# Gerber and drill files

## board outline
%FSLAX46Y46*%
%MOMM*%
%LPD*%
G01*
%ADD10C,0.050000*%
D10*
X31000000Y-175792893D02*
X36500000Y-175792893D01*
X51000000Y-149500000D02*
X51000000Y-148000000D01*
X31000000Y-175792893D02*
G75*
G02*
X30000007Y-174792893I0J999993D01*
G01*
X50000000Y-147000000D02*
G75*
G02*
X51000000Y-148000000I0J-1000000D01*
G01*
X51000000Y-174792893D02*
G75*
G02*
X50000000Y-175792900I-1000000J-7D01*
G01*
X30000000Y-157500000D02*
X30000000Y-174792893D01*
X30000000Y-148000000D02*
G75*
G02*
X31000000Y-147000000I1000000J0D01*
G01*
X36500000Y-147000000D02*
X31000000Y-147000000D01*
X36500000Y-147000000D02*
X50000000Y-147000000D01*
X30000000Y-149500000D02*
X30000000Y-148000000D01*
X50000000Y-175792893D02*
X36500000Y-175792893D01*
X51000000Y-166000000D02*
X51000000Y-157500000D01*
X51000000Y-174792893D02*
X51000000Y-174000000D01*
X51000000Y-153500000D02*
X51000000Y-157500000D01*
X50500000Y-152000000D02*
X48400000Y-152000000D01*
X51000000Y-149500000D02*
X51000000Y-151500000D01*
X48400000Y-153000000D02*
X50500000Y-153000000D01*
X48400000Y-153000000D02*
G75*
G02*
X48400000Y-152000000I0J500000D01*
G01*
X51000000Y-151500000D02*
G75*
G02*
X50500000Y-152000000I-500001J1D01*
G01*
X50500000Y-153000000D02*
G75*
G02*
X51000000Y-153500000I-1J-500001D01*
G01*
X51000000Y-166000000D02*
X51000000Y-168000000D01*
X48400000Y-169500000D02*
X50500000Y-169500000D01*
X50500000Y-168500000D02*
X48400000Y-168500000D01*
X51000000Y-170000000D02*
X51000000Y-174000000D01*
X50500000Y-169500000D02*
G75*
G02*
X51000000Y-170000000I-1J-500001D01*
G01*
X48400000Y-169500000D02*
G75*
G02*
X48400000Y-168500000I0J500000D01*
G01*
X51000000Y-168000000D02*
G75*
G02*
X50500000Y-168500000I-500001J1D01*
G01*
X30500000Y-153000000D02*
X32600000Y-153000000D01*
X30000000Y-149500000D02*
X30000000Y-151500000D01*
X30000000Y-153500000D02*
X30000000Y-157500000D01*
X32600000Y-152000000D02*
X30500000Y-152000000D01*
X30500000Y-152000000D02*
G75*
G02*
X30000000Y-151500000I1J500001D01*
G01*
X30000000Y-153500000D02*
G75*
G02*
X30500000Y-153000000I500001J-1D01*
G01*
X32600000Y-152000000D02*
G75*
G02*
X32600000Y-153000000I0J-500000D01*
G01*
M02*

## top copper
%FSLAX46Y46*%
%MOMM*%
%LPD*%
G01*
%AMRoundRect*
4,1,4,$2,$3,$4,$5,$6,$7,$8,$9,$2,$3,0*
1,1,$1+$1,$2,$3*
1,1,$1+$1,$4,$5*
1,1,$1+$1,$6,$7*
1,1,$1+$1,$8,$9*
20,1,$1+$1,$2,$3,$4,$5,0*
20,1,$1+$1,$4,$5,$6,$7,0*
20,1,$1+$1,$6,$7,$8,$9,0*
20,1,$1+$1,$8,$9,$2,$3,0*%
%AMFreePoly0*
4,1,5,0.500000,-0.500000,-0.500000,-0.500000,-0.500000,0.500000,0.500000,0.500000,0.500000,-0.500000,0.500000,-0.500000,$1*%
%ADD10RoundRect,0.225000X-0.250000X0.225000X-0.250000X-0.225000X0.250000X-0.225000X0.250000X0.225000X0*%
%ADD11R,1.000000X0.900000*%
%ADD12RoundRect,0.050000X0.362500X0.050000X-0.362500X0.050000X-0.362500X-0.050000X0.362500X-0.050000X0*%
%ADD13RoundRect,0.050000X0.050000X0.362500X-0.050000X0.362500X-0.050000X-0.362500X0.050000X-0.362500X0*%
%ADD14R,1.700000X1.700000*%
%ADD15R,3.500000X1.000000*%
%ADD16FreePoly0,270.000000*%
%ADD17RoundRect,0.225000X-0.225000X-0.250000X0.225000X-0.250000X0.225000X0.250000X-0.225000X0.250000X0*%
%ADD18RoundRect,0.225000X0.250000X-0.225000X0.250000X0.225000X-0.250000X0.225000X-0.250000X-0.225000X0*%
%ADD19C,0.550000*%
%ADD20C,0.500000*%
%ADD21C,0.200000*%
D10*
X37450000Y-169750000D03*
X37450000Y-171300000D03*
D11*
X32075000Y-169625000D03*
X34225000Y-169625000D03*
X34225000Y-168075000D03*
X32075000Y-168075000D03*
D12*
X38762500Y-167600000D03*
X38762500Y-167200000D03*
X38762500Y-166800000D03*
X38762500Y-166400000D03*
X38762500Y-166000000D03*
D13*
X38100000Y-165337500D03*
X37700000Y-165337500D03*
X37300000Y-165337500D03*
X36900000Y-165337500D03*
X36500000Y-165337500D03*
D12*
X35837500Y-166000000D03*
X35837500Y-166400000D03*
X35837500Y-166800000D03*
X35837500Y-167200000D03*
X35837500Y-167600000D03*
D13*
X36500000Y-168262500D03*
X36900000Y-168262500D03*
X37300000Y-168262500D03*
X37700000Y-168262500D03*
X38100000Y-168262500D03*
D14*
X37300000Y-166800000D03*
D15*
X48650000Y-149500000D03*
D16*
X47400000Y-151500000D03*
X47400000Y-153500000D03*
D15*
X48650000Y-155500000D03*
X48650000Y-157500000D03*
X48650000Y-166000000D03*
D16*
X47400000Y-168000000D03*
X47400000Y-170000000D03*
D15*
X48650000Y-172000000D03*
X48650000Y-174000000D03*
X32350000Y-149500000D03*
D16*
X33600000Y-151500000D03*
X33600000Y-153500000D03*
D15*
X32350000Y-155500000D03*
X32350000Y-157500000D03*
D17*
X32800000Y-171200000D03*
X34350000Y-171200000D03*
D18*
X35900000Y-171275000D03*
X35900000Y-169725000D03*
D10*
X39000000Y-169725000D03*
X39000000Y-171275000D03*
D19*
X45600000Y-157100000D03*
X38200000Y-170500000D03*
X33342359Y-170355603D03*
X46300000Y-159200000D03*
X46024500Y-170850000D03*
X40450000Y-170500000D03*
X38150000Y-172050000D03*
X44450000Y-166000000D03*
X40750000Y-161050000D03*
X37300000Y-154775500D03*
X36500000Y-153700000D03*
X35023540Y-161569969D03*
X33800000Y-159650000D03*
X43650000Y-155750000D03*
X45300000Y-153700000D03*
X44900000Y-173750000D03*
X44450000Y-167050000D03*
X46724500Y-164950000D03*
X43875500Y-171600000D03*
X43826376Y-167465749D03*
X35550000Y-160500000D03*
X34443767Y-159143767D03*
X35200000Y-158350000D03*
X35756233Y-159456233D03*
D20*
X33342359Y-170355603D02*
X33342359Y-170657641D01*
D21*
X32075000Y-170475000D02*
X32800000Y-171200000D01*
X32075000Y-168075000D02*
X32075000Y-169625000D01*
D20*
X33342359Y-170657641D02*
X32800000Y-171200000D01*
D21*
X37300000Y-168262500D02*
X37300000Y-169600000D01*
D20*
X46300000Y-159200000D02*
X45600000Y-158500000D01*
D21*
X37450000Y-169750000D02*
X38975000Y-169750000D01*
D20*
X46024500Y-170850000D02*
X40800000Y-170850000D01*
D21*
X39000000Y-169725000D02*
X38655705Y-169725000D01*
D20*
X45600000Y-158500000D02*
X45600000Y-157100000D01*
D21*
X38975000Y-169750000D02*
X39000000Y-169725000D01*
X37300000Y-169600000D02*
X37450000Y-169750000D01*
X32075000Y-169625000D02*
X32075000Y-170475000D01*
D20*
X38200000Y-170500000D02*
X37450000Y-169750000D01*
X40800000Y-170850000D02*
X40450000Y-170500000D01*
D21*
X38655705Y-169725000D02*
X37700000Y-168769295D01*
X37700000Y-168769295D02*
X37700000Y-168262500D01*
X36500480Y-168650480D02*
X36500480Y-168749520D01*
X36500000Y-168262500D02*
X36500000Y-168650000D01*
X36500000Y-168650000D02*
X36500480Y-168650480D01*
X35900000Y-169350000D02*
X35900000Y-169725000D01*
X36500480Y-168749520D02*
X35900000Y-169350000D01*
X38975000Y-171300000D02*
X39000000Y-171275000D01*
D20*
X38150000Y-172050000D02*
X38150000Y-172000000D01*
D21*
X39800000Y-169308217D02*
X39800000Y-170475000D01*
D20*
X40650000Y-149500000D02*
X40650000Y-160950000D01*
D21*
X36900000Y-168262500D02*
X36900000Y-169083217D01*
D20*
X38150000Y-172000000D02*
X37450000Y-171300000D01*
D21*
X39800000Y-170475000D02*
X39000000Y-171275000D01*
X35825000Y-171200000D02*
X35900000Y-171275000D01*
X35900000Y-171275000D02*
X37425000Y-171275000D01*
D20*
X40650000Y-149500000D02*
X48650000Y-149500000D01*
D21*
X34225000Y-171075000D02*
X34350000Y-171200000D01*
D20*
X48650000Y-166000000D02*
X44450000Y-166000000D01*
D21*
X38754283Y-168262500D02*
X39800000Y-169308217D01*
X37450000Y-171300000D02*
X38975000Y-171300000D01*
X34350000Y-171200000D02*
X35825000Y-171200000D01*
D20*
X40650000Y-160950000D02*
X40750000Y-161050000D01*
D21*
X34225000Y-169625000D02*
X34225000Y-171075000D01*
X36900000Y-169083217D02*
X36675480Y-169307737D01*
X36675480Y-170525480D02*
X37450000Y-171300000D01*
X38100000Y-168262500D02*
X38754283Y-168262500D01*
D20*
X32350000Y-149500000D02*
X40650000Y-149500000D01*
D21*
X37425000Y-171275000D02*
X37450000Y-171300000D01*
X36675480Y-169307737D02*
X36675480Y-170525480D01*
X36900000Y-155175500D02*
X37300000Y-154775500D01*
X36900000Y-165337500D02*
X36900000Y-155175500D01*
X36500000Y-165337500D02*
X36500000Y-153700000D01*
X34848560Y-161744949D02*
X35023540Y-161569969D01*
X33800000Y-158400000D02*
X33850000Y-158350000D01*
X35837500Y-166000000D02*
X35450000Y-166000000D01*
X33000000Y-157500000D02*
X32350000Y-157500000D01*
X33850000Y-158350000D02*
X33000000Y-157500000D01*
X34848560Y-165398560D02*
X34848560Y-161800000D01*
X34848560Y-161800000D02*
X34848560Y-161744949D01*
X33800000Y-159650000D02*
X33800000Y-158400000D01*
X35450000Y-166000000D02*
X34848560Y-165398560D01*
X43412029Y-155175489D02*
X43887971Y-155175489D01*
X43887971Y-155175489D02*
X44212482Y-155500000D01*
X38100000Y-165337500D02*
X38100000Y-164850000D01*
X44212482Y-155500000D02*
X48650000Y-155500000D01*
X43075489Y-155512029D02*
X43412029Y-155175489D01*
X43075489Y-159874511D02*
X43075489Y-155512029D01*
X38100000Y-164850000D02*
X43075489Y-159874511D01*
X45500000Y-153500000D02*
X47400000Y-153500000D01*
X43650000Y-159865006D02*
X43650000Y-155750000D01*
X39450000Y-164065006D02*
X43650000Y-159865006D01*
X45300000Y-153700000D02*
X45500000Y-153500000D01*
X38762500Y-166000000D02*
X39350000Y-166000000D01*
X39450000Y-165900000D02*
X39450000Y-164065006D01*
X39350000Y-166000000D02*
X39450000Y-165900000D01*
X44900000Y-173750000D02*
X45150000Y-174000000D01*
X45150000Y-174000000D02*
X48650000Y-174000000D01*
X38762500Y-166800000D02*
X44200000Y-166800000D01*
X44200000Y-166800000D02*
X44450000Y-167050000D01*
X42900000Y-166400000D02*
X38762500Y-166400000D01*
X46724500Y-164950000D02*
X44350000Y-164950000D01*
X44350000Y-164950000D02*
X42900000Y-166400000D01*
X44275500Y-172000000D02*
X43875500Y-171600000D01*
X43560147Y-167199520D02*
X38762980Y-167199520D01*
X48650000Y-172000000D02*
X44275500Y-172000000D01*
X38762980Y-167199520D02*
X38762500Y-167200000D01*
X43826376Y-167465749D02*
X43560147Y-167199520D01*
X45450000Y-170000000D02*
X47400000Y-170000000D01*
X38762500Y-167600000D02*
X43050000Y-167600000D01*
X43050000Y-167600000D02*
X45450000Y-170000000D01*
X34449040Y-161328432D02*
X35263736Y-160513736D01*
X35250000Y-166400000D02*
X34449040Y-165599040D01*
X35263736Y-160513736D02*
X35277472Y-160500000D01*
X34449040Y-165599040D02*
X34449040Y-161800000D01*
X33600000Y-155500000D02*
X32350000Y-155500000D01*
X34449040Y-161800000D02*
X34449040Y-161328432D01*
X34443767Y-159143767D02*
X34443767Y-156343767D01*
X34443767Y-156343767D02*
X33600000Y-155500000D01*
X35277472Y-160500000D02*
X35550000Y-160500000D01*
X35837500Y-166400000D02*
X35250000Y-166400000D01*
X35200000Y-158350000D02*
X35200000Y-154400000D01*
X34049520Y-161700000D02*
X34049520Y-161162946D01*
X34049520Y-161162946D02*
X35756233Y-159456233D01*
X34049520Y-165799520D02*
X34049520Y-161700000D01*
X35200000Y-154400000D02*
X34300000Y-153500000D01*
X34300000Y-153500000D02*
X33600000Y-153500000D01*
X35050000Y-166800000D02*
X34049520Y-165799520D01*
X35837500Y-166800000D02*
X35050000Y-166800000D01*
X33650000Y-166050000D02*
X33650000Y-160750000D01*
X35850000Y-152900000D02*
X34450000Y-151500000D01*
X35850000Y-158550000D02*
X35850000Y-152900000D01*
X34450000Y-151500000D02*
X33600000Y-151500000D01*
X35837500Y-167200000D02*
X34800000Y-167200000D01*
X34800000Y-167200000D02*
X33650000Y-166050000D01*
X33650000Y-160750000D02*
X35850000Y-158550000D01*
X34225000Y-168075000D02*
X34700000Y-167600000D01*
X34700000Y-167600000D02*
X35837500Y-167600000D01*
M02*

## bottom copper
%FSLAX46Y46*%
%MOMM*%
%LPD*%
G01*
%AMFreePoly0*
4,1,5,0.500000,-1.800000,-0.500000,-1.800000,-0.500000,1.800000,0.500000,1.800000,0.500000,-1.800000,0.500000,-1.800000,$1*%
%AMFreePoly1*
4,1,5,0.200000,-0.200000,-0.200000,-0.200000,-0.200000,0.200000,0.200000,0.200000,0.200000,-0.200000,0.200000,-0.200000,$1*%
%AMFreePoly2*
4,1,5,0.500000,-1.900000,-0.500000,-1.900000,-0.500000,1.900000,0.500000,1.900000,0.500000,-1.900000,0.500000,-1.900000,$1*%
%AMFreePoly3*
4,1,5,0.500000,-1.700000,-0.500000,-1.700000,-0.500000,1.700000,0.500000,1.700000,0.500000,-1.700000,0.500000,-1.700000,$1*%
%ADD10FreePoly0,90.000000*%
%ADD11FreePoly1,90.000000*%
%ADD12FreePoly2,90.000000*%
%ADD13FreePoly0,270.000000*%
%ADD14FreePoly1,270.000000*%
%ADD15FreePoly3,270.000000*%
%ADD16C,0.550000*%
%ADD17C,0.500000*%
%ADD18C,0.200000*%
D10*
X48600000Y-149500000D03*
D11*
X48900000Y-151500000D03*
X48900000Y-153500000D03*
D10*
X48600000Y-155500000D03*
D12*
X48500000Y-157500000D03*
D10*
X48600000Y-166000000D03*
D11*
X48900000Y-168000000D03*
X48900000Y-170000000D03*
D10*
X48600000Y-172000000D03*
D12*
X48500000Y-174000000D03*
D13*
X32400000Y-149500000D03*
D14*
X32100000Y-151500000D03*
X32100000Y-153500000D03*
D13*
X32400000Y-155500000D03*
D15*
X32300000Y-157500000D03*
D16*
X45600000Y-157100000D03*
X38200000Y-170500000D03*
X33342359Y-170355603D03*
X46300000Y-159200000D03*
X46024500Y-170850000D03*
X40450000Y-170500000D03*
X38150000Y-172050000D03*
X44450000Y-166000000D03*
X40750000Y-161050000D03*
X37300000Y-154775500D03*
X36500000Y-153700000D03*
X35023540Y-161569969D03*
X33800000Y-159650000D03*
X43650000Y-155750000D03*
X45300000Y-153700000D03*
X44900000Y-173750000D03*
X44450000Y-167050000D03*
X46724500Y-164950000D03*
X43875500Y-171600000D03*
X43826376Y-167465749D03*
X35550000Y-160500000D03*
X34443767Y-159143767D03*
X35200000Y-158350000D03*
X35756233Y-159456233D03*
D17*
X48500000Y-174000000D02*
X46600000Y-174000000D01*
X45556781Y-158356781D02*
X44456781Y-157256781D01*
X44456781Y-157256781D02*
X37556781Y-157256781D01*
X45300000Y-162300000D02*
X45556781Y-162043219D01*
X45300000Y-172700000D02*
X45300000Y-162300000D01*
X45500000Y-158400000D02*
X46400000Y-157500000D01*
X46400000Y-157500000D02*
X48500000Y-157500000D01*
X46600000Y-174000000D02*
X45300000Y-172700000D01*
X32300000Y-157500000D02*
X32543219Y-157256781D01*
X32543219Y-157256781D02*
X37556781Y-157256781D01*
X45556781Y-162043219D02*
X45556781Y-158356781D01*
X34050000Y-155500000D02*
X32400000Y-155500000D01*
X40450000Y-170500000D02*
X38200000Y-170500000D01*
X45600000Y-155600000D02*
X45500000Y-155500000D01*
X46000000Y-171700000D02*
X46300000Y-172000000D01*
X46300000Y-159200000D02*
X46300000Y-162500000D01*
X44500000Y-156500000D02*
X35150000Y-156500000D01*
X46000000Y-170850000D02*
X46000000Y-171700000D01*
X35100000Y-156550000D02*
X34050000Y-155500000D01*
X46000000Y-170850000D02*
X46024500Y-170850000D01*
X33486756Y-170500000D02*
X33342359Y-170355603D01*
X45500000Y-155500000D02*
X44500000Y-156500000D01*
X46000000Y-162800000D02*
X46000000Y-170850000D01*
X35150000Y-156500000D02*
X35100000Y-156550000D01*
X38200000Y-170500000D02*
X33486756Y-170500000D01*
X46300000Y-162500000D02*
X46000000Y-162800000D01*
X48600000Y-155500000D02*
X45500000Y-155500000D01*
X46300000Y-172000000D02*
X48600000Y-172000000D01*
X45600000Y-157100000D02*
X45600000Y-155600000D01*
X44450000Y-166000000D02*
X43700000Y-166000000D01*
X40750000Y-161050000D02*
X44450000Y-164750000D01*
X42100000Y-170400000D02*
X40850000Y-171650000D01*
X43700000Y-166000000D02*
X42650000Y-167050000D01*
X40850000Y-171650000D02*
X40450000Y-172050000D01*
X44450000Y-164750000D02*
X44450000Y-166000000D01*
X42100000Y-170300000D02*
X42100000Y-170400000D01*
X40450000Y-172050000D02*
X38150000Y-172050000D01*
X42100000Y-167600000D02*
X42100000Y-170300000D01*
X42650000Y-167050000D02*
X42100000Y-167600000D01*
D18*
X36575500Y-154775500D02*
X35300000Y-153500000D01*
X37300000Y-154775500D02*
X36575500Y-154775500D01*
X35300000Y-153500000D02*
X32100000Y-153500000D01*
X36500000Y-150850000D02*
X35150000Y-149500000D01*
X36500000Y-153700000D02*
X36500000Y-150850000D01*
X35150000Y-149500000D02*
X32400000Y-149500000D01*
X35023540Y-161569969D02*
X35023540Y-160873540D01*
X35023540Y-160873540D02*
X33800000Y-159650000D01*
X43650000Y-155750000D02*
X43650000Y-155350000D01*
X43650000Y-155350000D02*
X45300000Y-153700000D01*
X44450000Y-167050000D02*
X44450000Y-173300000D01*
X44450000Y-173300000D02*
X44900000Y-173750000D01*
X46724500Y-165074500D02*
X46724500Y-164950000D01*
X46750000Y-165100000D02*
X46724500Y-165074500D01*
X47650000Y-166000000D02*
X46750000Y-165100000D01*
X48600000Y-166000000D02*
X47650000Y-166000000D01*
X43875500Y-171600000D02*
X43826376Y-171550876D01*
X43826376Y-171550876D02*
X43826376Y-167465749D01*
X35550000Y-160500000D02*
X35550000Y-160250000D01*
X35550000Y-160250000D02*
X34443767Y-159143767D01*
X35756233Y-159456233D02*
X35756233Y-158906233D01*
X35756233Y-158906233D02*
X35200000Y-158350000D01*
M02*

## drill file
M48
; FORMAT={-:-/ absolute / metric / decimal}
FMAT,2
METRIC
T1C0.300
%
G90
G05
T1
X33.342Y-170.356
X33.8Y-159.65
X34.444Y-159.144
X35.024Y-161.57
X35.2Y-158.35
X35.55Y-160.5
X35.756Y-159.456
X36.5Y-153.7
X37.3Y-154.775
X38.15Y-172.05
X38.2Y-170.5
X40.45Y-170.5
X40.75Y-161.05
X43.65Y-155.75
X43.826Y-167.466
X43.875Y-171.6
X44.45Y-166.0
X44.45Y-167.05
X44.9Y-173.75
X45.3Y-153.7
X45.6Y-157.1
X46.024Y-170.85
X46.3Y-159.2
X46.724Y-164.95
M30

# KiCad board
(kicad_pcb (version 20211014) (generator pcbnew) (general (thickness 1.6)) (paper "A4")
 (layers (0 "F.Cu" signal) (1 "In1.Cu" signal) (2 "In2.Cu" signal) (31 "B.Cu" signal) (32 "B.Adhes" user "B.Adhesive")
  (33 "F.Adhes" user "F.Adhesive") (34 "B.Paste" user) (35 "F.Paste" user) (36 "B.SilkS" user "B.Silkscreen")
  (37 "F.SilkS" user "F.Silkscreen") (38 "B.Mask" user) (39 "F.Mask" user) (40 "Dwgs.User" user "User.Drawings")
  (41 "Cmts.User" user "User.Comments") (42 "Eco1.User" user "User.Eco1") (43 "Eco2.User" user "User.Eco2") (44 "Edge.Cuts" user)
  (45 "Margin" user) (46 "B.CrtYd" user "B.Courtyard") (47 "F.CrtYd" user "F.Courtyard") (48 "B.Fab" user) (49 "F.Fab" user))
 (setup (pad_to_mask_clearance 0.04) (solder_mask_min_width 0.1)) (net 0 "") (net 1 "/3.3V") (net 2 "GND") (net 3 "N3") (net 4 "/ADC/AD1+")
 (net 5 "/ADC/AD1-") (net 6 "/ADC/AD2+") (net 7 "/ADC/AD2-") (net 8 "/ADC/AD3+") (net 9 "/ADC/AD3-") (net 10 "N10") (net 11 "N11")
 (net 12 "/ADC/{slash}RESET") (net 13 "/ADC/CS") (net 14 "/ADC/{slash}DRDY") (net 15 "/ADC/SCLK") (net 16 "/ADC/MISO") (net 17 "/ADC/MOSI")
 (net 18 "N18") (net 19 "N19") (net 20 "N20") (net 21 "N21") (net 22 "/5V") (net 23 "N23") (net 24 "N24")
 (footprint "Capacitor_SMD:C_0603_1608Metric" (layer "F.Cu") (at 37.45 170.525 -90)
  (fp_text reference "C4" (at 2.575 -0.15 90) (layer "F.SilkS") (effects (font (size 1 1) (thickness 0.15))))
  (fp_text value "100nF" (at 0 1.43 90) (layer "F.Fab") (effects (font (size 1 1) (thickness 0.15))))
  (pad "1" smd roundrect locked (at -0.775 0 270) (size 0.9 0.95) (layers "F.Cu" "F.Paste" "F.Mask") (roundrect_rratio 0.25) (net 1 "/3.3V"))
  (pad "2" smd roundrect locked (at 0.775 0 270) (size 0.9 0.95) (layers "F.Cu" "F.Paste" "F.Mask") (roundrect_rratio 0.25) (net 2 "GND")))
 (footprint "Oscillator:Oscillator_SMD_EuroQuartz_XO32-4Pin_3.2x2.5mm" (layer "F.Cu") (at 33.15 168.85 90)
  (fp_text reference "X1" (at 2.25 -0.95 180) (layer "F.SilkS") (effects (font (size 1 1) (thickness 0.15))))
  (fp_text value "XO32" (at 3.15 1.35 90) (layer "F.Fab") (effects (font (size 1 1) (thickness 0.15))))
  (pad "1" smd rect locked (at -0.775 -1.075) (size 1 0.9) (layers "F.Cu" "F.Paste" "F.Mask") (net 1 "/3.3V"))
  (pad "2" smd rect locked (at -0.775 1.075) (size 1 0.9) (layers "F.Cu" "F.Paste" "F.Mask") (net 2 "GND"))
  (pad "3" smd rect locked (at 0.775 1.075) (size 1 0.9) (layers "F.Cu" "F.Paste" "F.Mask") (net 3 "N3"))
  (pad "4" smd rect locked (at 0.775 -1.075) (size 1 0.9) (layers "F.Cu" "F.Paste" "F.Mask") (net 1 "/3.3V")))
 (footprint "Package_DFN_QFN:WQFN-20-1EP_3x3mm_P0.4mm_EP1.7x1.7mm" (layer "F.Cu") (at 37.3 166.8 180)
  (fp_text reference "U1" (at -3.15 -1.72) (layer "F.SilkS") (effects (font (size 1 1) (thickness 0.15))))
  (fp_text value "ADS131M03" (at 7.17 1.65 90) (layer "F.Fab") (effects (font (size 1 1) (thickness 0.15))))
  (pad "" smd roundrect locked (at -0.425 0.425 180) (size 0.69 0.69) (layers "F.Paste") (roundrect_rratio 0.25))
  (pad "" smd roundrect locked (at 0.425 -0.425 180) (size 0.69 0.69) (layers "F.Paste") (roundrect_rratio 0.25))
  (pad "" smd roundrect locked (at 0.425 0.425 180) (size 0.69 0.69) (layers "F.Paste") (roundrect_rratio 0.25))
  (pad "" smd roundrect locked (at -0.425 -0.425 180) (size 0.69 0.69) (layers "F.Paste") (roundrect_rratio 0.25))
  (pad "1" smd roundrect locked (at -1.4625 -0.8 180) (size 0.825 0.2) (layers "F.Cu" "F.Paste" "F.Mask") (roundrect_rratio 0.25)
   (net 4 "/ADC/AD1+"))
  (pad "2" smd roundrect locked (at -1.4625 -0.4 180) (size 0.825 0.2) (layers "F.Cu" "F.Paste" "F.Mask") (roundrect_rratio 0.25)
   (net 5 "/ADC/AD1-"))
  (pad "3" smd roundrect locked (at -1.4625 0 180) (size 0.825 0.2) (layers "F.Cu" "F.Paste" "F.Mask") (roundrect_rratio 0.25)
   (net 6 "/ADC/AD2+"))
  (pad "4" smd roundrect locked (at -1.4625 0.4 180) (size 0.825 0.2) (layers "F.Cu" "F.Paste" "F.Mask") (roundrect_rratio 0.25)
   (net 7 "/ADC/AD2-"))
  (pad "5" smd roundrect locked (at -1.4625 0.8 180) (size 0.825 0.2) (layers "F.Cu" "F.Paste" "F.Mask") (roundrect_rratio 0.25)
   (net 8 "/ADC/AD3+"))
  (pad "6" smd roundrect locked (at -0.8 1.4625 180) (size 0.2 0.825) (layers "F.Cu" "F.Paste" "F.Mask") (roundrect_rratio 0.25)
   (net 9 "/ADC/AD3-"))
  (pad "7" smd roundrect locked (at -0.4 1.4625 180) (size 0.2 0.825) (layers "F.Cu" "F.Paste" "F.Mask") (roundrect_rratio 0.25)
   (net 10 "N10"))
  (pad "8" smd roundrect locked (at 0 1.4625 180) (size 0.2 0.825) (layers "F.Cu" "F.Paste" "F.Mask") (roundrect_rratio 0.25) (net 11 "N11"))
  (pad "9" smd roundrect locked (at 0.4 1.4625 180) (size 0.2 0.825) (layers "F.Cu" "F.Paste" "F.Mask") (roundrect_rratio 0.25)
   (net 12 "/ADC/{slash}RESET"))
  (pad "10" smd roundrect locked (at 0.8 1.4625 180) (size 0.2 0.825) (layers "F.Cu" "F.Paste" "F.Mask") (roundrect_rratio 0.25)
   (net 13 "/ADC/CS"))
  (pad "11" smd roundrect locked (at 1.4625 0.8 180) (size 0.825 0.2) (layers "F.Cu" "F.Paste" "F.Mask") (roundrect_rratio 0.25)
   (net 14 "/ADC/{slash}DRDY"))
  (pad "12" smd roundrect locked (at 1.4625 0.4 180) (size 0.825 0.2) (layers "F.Cu" "F.Paste" "F.Mask") (roundrect_rratio 0.25)
   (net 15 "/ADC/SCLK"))
  (pad "13" smd roundrect locked (at 1.4625 0 180) (size 0.825 0.2) (layers "F.Cu" "F.Paste" "F.Mask") (roundrect_rratio 0.25)
   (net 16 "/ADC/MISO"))
  (pad "14" smd roundrect locked (at 1.4625 -0.4 180) (size 0.825 0.2) (layers "F.Cu" "F.Paste" "F.Mask") (roundrect_rratio 0.25)
   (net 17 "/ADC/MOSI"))
  (pad "15" smd roundrect locked (at 1.4625 -0.8 180) (size 0.825 0.2) (layers "F.Cu" "F.Paste" "F.Mask") (roundrect_rratio 0.25)
   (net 3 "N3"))
  (pad "16" smd roundrect locked (at 0.8 -1.4625 180) (size 0.2 0.825) (layers "F.Cu" "F.Paste" "F.Mask") (roundrect_rratio 0.25)
   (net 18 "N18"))
  (pad "17" smd roundrect locked (at 0.4 -1.4625 180) (size 0.2 0.825) (layers "F.Cu" "F.Paste" "F.Mask") (roundrect_rratio 0.25)
   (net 2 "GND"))
  (pad "18" smd roundrect locked (at 0 -1.4625 180) (size 0.2 0.825) (layers "F.Cu" "F.Paste" "F.Mask") (roundrect_rratio 0.25)
   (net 1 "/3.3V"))
  (pad "19" smd roundrect locked (at -0.4 -1.4625 180) (size 0.2 0.825) (layers "F.Cu" "F.Paste" "F.Mask") (roundrect_rratio 0.25)
   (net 1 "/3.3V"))
  (pad "20" smd roundrect locked (at -0.8 -1.4625 180) (size 0.2 0.825) (layers "F.Cu" "F.Paste" "F.Mask") (roundrect_rratio 0.25)
   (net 2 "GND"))
  (pad "21" smd rect locked (at 0 0 180) (size 1.7 1.7) (layers "F.Cu" "F.Mask")))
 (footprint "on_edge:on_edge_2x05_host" (layer "F.Cu") (at 51 153.5 -90)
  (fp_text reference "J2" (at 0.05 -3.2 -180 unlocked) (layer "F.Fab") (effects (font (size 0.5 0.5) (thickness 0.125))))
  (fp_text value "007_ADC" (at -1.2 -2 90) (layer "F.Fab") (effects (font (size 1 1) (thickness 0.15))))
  (fp_line (start 0 0) (end 4 0) (layer "Edge.Cuts") (width 0.05))
  (fp_line (start -1.5 0.5) (end -1.5 2.6) (layer "Edge.Cuts") (width 0.05))
  (fp_line (start -4 0) (end -2 0) (layer "Edge.Cuts") (width 0.05))
  (fp_line (start -0.5 2.6) (end -0.5 0.5) (layer "Edge.Cuts") (width 0.05))
  (fp_arc (start -0.5 2.6) (mid -1 3.1) (end -1.5 2.6) (layer "Edge.Cuts") (width 0.05))
  (fp_arc (start -2 0) (mid -1.646447 0.146447) (end -1.5 0.5) (layer "Edge.Cuts") (width 0.05))
  (fp_arc (start -0.5 0.5) (mid -0.353553 0.146447) (end 0 0) (layer "Edge.Cuts") (width 0.05))
  (pad "1" smd rect locked (at -4 2.35 270) (size 1 3.5) (layers "F.Cu" "F.Mask") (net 2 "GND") (zone_connect 0))
  (pad "2" smd custom locked (at -2 3.6 270) (size 1 1) (layers "F.Cu" "F.Mask") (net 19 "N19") (zone_connect 0)
   (options (clearance outline) (anchor rect)) (primitives))
  (pad "3" smd custom locked (at 0 3.6 270) (size 1 1) (layers "F.Cu" "F.Mask") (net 8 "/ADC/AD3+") (zone_connect 0)
   (options (clearance outline) (anchor rect)) (primitives))
  (pad "4" smd rect locked (at 2 2.35 270) (size 1 3.5) (layers "F.Cu" "F.Mask") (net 9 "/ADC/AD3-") (zone_connect 0))
  (pad "5" smd rect locked (at 4 2.35 270) (size 1 3.5) (layers "F.Cu" "F.Mask") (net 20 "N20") (zone_connect 0))
  (pad "6" smd custom locked (at -4 2.4 90) (size 1 3.6) (layers "B.Cu" "B.Mask") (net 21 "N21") (zone_connect 0)
   (options (clearance outline) (anchor rect)) (primitives))
  (pad "7" smd custom locked (at -2 2.1 90) (size 0.4 0.4) (layers "B.Cu" "B.Mask") (zone_connect 0)
   (options (clearance outline) (anchor rect)) (primitives))
  (pad "8" smd custom locked (at 0 2.1 90) (size 0.4 0.4) (layers "B.Cu" "B.Mask") (zone_connect 0)
   (options (clearance outline) (anchor rect)) (primitives))
  (pad "9" smd custom locked (at 2 2.4 90) (size 1 3.6) (layers "B.Cu" "B.Mask") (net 1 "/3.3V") (zone_connect 0)
   (options (clearance outline) (anchor rect)) (primitives))
  (pad "10" smd custom locked (at 4 2.5 90) (size 1 3.8) (layers "B.Cu" "B.Mask") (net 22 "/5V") (zone_connect 0)
   (options (clearance outline) (anchor rect)) (primitives)))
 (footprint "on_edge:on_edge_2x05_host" (layer "F.Cu") (at 51 170 -90)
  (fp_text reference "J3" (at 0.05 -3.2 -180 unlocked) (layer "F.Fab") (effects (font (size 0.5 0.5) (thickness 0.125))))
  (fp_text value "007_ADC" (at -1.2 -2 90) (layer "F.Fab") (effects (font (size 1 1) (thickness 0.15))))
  (fp_line (start -4 0) (end -2 0) (layer "Edge.Cuts") (width 0.05))
  (fp_line (start -0.5 2.6) (end -0.5 0.5) (layer "Edge.Cuts") (width 0.05))
  (fp_line (start -1.5 0.5) (end -1.5 2.6) (layer "Edge.Cuts") (width 0.05))
  (fp_line (start 0 0) (end 4 0) (layer "Edge.Cuts") (width 0.05))
  (fp_arc (start -0.5 0.5) (mid -0.353553 0.146447) (end 0 0) (layer "Edge.Cuts") (width 0.05))
  (fp_arc (start -0.5 2.6) (mid -1 3.1) (end -1.5 2.6) (layer "Edge.Cuts") (width 0.05))
  (fp_arc (start -2 0) (mid -1.646447 0.146447) (end -1.5 0.5) (layer "Edge.Cuts") (width 0.05))
  (pad "1" smd rect locked (at -4 2.35 270) (size 1 3.5) (layers "F.Cu" "F.Mask") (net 2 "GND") (zone_connect 0))
  (pad "2" smd custom locked (at -2 3.6 270) (size 1 1) (layers "F.Cu" "F.Mask") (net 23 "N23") (zone_connect 0)
   (options (clearance outline) (anchor rect)) (primitives))
  (pad "3" smd custom locked (at 0 3.6 270) (size 1 1) (layers "F.Cu" "F.Mask") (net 4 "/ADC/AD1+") (zone_connect 0)
   (options (clearance outline) (anchor rect)) (primitives))
  (pad "4" smd rect locked (at 2 2.35 270) (size 1 3.5) (layers "F.Cu" "F.Mask") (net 5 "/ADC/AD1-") (zone_connect 0))
  (pad "5" smd rect locked (at 4 2.35 270) (size 1 3.5) (layers "F.Cu" "F.Mask") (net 6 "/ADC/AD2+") (zone_connect 0))
  (pad "6" smd custom locked (at -4 2.4 90) (size 1 3.6) (layers "B.Cu" "B.Mask") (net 7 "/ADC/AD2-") (zone_connect 0)
   (options (clearance outline) (anchor rect)) (primitives))
  (pad "7" smd custom locked (at -2 2.1 90) (size 0.4 0.4) (layers "B.Cu" "B.Mask") (zone_connect 0)
   (options (clearance outline) (anchor rect)) (primitives))
  (pad "8" smd custom locked (at 0 2.1 90) (size 0.4 0.4) (layers "B.Cu" "B.Mask") (zone_connect 0)
   (options (clearance outline) (anchor rect)) (primitives))
  (pad "9" smd custom locked (at 2 2.4 90) (size 1 3.6) (layers "B.Cu" "B.Mask") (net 1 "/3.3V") (zone_connect 0)
   (options (clearance outline) (anchor rect)) (primitives))
  (pad "10" smd custom locked (at 4 2.5 90) (size 1 3.8) (layers "B.Cu" "B.Mask") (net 22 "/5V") (zone_connect 0)
   (options (clearance outline) (anchor rect)) (primitives)))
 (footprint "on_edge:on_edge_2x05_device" (layer "F.Cu") (at 30 153.5 -90)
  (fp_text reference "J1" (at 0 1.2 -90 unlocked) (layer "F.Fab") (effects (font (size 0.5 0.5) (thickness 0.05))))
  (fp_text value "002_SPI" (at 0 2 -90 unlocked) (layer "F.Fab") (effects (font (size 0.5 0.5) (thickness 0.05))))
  (fp_line (start -0.5 -0.5) (end -0.5 -2.6) (layer "Edge.Cuts") (width 0.05))
  (fp_line (start -4 0) (end -2 0) (layer "Edge.Cuts") (width 0.05))
  (fp_line (start 0 0) (end 4 0) (layer "Edge.Cuts") (width 0.05))
  (fp_line (start -1.5 -2.6) (end -1.5 -0.5) (layer "Edge.Cuts") (width 0.05))
  (fp_arc (start -1.5 -0.5) (mid -1.646447 -0.146447) (end -2 0) (layer "Edge.Cuts") (width 0.05))
  (fp_arc (start 0 0) (mid -0.353553 -0.146447) (end -0.5 -0.5) (layer "Edge.Cuts") (width 0.05))
  (fp_arc (start -1.5 -2.6) (mid -1 -3.1) (end -0.5 -2.6) (layer "Edge.Cuts") (width 0.05))
  (pad "1" smd rect locked (at -4 -2.35 90) (size 1 3.5) (layers "F.Cu" "F.Mask") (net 2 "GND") (zone_connect 0))
  (pad "2" smd custom locked (at -2 -3.6 270) (size 1 1) (layers "F.Cu" "F.Mask") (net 17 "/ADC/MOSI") (zone_connect 0)
   (options (clearance outline) (anchor rect)) (primitives))
  (pad "3" smd custom locked (at 0 -3.6 270) (size 1 1) (layers "F.Cu" "F.Mask") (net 16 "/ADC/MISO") (zone_connect 0)
   (options (clearance outline) (anchor rect)) (primitives))
  (pad "4" smd rect locked (at 2 -2.35 90) (size 1 3.5) (layers "F.Cu" "F.Mask") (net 15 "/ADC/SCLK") (zone_connect 0))
  (pad "5" smd rect locked (at 4 -2.35 90) (size 1 3.5) (layers "F.Cu" "F.Mask") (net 14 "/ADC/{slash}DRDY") (zone_connect 0))
  (pad "6" smd custom locked (at -4 -2.4 270) (size 1 3.6) (layers "B.Cu" "B.Mask") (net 13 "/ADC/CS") (zone_connect 0)
   (options (clearance outline) (anchor rect)) (primitives))
  (pad "7" smd custom locked (at -2 -2.1 270) (size 0.4 0.4) (layers "B.Cu" "B.Mask") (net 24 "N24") (zone_connect 0)
   (options (clearance outline) (anchor rect)) (primitives))
  (pad "8" smd custom locked (at 0 -2.1 270) (size 0.4 0.4) (layers "B.Cu" "B.Mask") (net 12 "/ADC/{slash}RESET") (zone_connect 0)
   (options (clearance outline) (anchor rect)) (primitives))
  (pad "9" smd custom locked (at 2 -2.4 270) (size 1 3.6) (layers "B.Cu" "B.Mask") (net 1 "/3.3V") (zone_connect 0)
   (options (clearance outline) (anchor rect)) (primitives))
  (pad "10" smd custom locked (at 4 -2.3 270) (size 1 3.4) (layers "B.Cu" "B.Mask") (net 22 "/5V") (zone_connect 0)
   (options (clearance outline) (anchor rect)) (primitives)))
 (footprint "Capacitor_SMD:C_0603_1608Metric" (layer "F.Cu") (at 33.575 171.2)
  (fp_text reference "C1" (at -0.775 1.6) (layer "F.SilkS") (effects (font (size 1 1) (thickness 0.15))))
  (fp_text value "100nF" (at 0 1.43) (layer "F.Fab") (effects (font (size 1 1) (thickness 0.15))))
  (pad "1" smd roundrect locked (at -0.775 0) (size 0.9 0.95) (layers "F.Cu" "F.Paste" "F.Mask") (roundrect_rratio 0.25) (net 1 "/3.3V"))
  (pad "2" smd roundrect locked (at 0.775 0) (size 0.9 0.95) (layers "F.Cu" "F.Paste" "F.Mask") (roundrect_rratio 0.25) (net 2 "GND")))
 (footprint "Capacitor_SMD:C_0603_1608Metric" (layer "F.Cu") (at 35.9 170.5 90)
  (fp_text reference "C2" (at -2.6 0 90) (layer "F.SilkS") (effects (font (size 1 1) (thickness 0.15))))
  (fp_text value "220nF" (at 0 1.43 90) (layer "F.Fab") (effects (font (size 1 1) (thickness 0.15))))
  (pad "1" smd roundrect locked (at -0.775 0 90) (size 0.9 0.95) (layers "F.Cu" "F.Paste" "F.Mask") (roundrect_rratio 0.25) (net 2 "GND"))
  (pad "2" smd roundrect locked (at 0.775 0 90) (size 0.9 0.95) (layers "F.Cu" "F.Paste" "F.Mask") (roundrect_rratio 0.25) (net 18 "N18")))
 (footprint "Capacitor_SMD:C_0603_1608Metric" (layer "F.Cu") (at 39 170.5 -90)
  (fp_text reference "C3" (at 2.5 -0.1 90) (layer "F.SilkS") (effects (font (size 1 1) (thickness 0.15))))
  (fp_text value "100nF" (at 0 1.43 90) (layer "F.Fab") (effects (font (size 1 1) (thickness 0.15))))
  (pad "1" smd roundrect locked (at -0.775 0 270) (size 0.9 0.95) (layers "F.Cu" "F.Paste" "F.Mask") (roundrect_rratio 0.25) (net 1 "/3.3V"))
  (pad "2" smd roundrect locked (at 0.775 0 270) (size 0.9 0.95) (layers "F.Cu" "F.Paste" "F.Mask") (roundrect_rratio 0.25) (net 2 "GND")))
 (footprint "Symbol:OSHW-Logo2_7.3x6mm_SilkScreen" (layer "B.Cu") (at 40.4 172.892893 180)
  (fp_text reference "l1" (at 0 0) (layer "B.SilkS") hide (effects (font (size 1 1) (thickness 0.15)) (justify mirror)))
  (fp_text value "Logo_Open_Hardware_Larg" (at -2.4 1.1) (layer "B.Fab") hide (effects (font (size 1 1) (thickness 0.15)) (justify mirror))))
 (gr_line (start 31 175.792893) (end 36.5 175.792893) (layer "Edge.Cuts") (width 0.05))
 (gr_line (start 51 149.5) (end 51 148) (layer "Edge.Cuts") (width 0.05))
 (gr_arc (start 31 175.792893) (mid 30.292893 175.5) (end 30 174.792893) (layer "Edge.Cuts") (width 0.05))
 (gr_arc (start 50 147) (mid 50.707107 147.292893) (end 51 148) (layer "Edge.Cuts") (width 0.05))
 (gr_arc (start 51 174.792893) (mid 50.707107 175.5) (end 50 175.792893) (layer "Edge.Cuts") (width 0.05))
 (gr_line (start 30 157.5) (end 30 174.792893) (layer "Edge.Cuts") (width 0.05))
 (gr_arc (start 30 148) (mid 30.292893 147.292893) (end 31 147) (layer "Edge.Cuts") (width 0.05))
 (gr_line (start 36.5 147) (end 31 147) (layer "Edge.Cuts") (width 0.05))
 (gr_line (start 36.5 147) (end 50 147) (layer "Edge.Cuts") (width 0.05))
 (gr_line (start 30 149.5) (end 30 148) (layer "Edge.Cuts") (width 0.05))
 (gr_line (start 50 175.792893) (end 36.5 175.792893) (layer "Edge.Cuts") (width 0.05))
 (gr_line (start 51 166) (end 51 157.5) (layer "Edge.Cuts") (width 0.05))
 (gr_line (start 51 174.792893) (end 51 174) (layer "Edge.Cuts") (width 0.05))
 (segment (start 48.5 174) (end 46.6 174) (width 0.5) (layer "B.Cu") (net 22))
 (segment (start 45.556781 158.356781) (end 44.456781 157.256781) (width 0.5) (layer "B.Cu") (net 22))
 (segment (start 44.456781 157.256781) (end 37.556781 157.256781) (width 0.5) (layer "B.Cu") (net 22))
 (segment (start 45.3 162.3) (end 45.556781 162.043219) (width 0.5) (layer "B.Cu") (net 22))
 (segment (start 45.3 172.7) (end 45.3 162.3) (width 0.5) (layer "B.Cu") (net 22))
 (segment (start 45.5 158.4) (end 46.4 157.5) (width 0.5) (layer "B.Cu") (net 22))
 (segment (start 46.4 157.5) (end 48.5 157.5) (width 0.5) (layer "B.Cu") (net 22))
 (segment (start 46.6 174) (end 45.3 172.7) (width 0.5) (layer "B.Cu") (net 22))
 (segment (start 32.3 157.5) (end 32.543219 157.256781) (width 0.5) (layer "B.Cu") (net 22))
 (segment (start 32.543219 157.256781) (end 37.556781 157.256781) (width 0.5) (layer "B.Cu") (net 22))
 (segment (start 45.556781 162.043219) (end 45.556781 158.356781) (width 0.5) (layer "B.Cu") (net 22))
 (segment (start 33.342359 170.355603) (end 33.342359 170.657641) (width 0.5) (layer "F.Cu") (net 1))
 (segment (start 32.075 170.475) (end 32.8 171.2) (width 0.2) (layer "F.Cu") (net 1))
 (segment (start 32.075 168.075) (end 32.075 169.625) (width 0.2) (layer "F.Cu") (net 1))
 (segment (start 33.342359 170.657641) (end 32.8 171.2) (width 0.5) (layer "F.Cu") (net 1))
 (segment (start 37.3 168.2625) (end 37.3 169.6) (width 0.2) (layer "F.Cu") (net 1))
 (segment (start 46.3 159.2) (end 45.6 158.5) (width 0.5) (layer "F.Cu") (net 1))
 (segment (start 37.45 169.75) (end 38.975 169.75) (width 0.2) (layer "F.Cu") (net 1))
 (segment (start 46.0245 170.85) (end 40.8 170.85) (width 0.5) (layer "F.Cu") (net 1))
 (segment (start 39 169.725) (end 38.655705 169.725) (width 0.2) (layer "F.Cu") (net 1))
 (segment (start 45.6 158.5) (end 45.6 157.1) (width 0.5) (layer "F.Cu") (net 1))
 (segment (start 38.975 169.75) (end 39 169.725) (width 0.2) (layer "F.Cu") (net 1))
 (segment (start 37.3 169.6) (end 37.45 169.75) (width 0.2) (layer "F.Cu") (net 1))
 (segment (start 32.075 169.625) (end 32.075 170.475) (width 0.2) (layer "F.Cu") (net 1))
 (segment (start 38.2 170.5) (end 37.45 169.75) (width 0.5) (layer "F.Cu") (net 1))
 (segment (start 40.8 170.85) (end 40.45 170.5) (width 0.5) (layer "F.Cu") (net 1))
 (segment (start 38.655705 169.725) (end 37.7 168.769295) (width 0.2) (layer "F.Cu") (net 1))
 (segment (start 37.7 168.769295) (end 37.7 168.2625) (width 0.2) (layer "F.Cu") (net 1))
 (via (at 45.6 157.1) (size 0.55) (drill 0.3) (layers "F.Cu" "B.Cu") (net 1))
 (via (at 38.2 170.5) (size 0.55) (drill 0.3) (layers "F.Cu" "B.Cu") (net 1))
 (via (at 33.342359 170.355603) (size 0.55) (drill 0.3) (layers "F.Cu" "B.Cu") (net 1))
 (via (at 46.3 159.2) (size 0.55) (drill 0.3) (layers "F.Cu" "B.Cu") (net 1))
 (via (at 46.0245 170.85) (size 0.55) (drill 0.3) (layers "F.Cu" "B.Cu") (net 1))
 (via (at 40.45 170.5) (size 0.55) (drill 0.3) (layers "F.Cu" "B.Cu") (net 1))
 (segment (start 34.05 155.5) (end 32.4 155.5) (width 0.5) (layer "B.Cu") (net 1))
 (segment (start 40.45 170.5) (end 38.2 170.5) (width 0.5) (layer "B.Cu") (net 1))
 (segment (start 45.6 155.6) (end 45.5 155.5) (width 0.5) (layer "B.Cu") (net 1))
 (segment (start 46 171.7) (end 46.3 172) (width 0.5) (layer "B.Cu") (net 1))
 (segment (start 46.3 159.2) (end 46.3 162.5) (width 0.5) (layer "B.Cu") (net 1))
 (segment (start 44.5 156.5) (end 35.15 156.5) (width 0.5) (layer "B.Cu") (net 1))
 (segment (start 46 170.85) (end 46 171.7) (width 0.5) (layer "B.Cu") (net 1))
 (segment (start 35.1 156.55) (end 34.05 155.5) (width 0.5) (layer "B.Cu") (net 1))
 (segment (start 46 170.85) (end 46.0245 170.85) (width 0.5) (layer "B.Cu") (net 1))
 (segment (start 33.486756 170.5) (end 33.342359 170.355603) (width 0.5) (layer "B.Cu") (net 1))
 (segment (start 45.5 155.5) (end 44.5 156.5) (width 0.5) (layer "B.Cu") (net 1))
 (segment (start 46 162.8) (end 46 170.85) (width 0.5) (layer "B.Cu") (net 1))
 (segment (start 35.15 156.5) (end 35.1 156.55) (width 0.5) (layer "B.Cu") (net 1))
 (segment (start 38.2 170.5) (end 33.486756 170.5) (width 0.5) (layer "B.Cu") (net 1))
 (segment (start 46.3 162.5) (end 46 162.8) (width 0.5) (layer "B.Cu") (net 1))
 (segment (start 48.6 155.5) (end 45.5 155.5) (width 0.5) (layer "B.Cu") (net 1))
 (segment (start 46.3 172) (end 48.6 172) (width 0.5) (layer "B.Cu") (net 1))
 (segment (start 45.6 157.1) (end 45.6 155.6) (width 0.5) (layer "B.Cu") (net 1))
 (segment (start 36.50048 168.65048) (end 36.50048 168.74952) (width 0.2) (layer "F.Cu") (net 18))
 (segment (start 36.5 168.2625) (end 36.5 168.65) (width 0.2) (layer "F.Cu") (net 18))
 (segment (start 36.5 168.65) (end 36.50048 168.65048) (width 0.2) (layer "F.Cu") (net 18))
 (segment (start 35.9 169.35) (end 35.9 169.725) (width 0.2) (layer "F.Cu") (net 18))
 (segment (start 36.50048 168.74952) (end 35.9 169.35) (width 0.2) (layer "F.Cu") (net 18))
 (segment (start 38.975 171.3) (end 39 171.275) (width 0.2) (layer "F.Cu") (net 2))
 (segment (start 38.15 172.05) (end 38.15 172) (width 0.5) (layer "F.Cu") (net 2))
 (segment (start 39.8 169.308217) (end 39.8 170.475) (width 0.2) (layer "F.Cu") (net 2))
 (segment (start 40.65 149.5) (end 40.65 160.95) (width 0.5) (layer "F.Cu") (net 2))
 (segment (start 36.9 168.2625) (end 36.9 169.083217) (width 0.2) (layer "F.Cu") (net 2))
 (segment (start 38.15 172) (end 37.45 171.3) (width 0.5) (layer "F.Cu") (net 2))
 (segment (start 39.8 170.475) (end 39 171.275) (width 0.2) (layer "F.Cu") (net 2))
 (segment (start 35.825 171.2) (end 35.9 171.275) (width 0.2) (layer "F.Cu") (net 2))
 (segment (start 35.9 171.275) (end 37.425 171.275) (width 0.2) (layer "F.Cu") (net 2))
 (segment (start 40.65 149.5) (end 48.65 149.5) (width 0.5) (layer "F.Cu") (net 2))
 (segment (start 34.225 171.075) (end 34.35 171.2) (width 0.2) (layer "F.Cu") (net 2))
 (segment (start 48.65 166) (end 44.45 166) (width 0.5) (layer "F.Cu") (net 2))
 (segment (start 38.754283 168.2625) (end 39.8 169.308217) (width 0.2) (layer "F.Cu") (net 2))
 (segment (start 37.45 171.3) (end 38.975 171.3) (width 0.2) (layer "F.Cu") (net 2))
 (segment (start 34.35 171.2) (end 35.825 171.2) (width 0.2) (layer "F.Cu") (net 2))
 (segment (start 40.65 160.95) (end 40.75 161.05) (width 0.5) (layer "F.Cu") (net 2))
 (segment (start 34.225 169.625) (end 34.225 171.075) (width 0.2) (layer "F.Cu") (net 2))
 (segment (start 36.9 169.083217) (end 36.67548 169.307737) (width 0.2) (layer "F.Cu") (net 2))
 (segment (start 36.67548 170.52548) (end 37.45 171.3) (width 0.2) (layer "F.Cu") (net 2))
 (segment (start 38.1 168.2625) (end 38.754283 168.2625) (width 0.2) (layer "F.Cu") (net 2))
 (segment (start 32.35 149.5) (end 40.65 149.5) (width 0.5) (layer "F.Cu") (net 2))
 (segment (start 37.425 171.275) (end 37.45 171.3) (width 0.2) (layer "F.Cu") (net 2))
 (segment (start 36.67548 169.307737) (end 36.67548 170.52548) (width 0.2) (layer "F.Cu") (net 2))
 (via (at 38.15 172.05) (size 0.55) (drill 0.3) (layers "F.Cu" "B.Cu") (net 2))
 (via (at 44.45 166) (size 0.55) (drill 0.3) (layers "F.Cu" "B.Cu") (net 2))
 (via (at 40.75 161.05) (size 0.55) (drill 0.3) (layers "F.Cu" "B.Cu") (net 2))
 (segment (start 44.45 166) (end 43.7 166) (width 0.5) (layer "B.Cu") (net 2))
 (segment (start 40.75 161.05) (end 44.45 164.75) (width 0.5) (layer "B.Cu") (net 2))
 (segment (start 42.1 170.4) (end 40.85 171.65) (width 0.5) (layer "B.Cu") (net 2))
 (segment (start 43.7 166) (end 42.65 167.05) (width 0.5) (layer "B.Cu") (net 2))
 (segment (start 40.85 171.65) (end 40.45 172.05) (width 0.5) (layer "B.Cu") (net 2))
 (segment (start 44.45 164.75) (end 44.45 166) (width 0.5) (layer "B.Cu") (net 2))
 (segment (start 42.1 170.3) (end 42.1 170.4) (width 0.5) (layer "B.Cu") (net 2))
 (segment (start 40.45 172.05) (end 38.15 172.05) (width 0.5) (layer "B.Cu") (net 2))
 (segment (start 42.1 167.6) (end 42.1 170.3) (width 0.5) (layer "B.Cu") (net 2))
 (segment (start 42.65 167.05) (end 42.1 167.6) (width 0.5) (layer "B.Cu") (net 2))
 (segment (start 36.9 155.1755) (end 37.3 154.7755) (width 0.2) (layer "F.Cu") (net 12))
 (segment (start 36.9 165.3375) (end 36.9 155.1755) (width 0.2) (layer "F.Cu") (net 12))
 (via (at 37.3 154.7755) (size 0.55) (drill 0.3) (layers "F.Cu" "B.Cu") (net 12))
 (segment (start 36.5755 154.7755) (end 35.3 153.5) (width 0.2) (layer "B.Cu") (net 12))
 (segment (start 37.3 154.7755) (end 36.5755 154.7755) (width 0.2) (layer "B.Cu") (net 12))
 (segment (start 35.3 153.5) (end 32.1 153.5) (width 0.2) (layer "B.Cu") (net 12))
 (segment (start 36.5 165.3375) (end 36.5 153.7) (width 0.2) (layer "F.Cu") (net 13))
 (via (at 36.5 153.7) (size 0.55) (drill 0.3) (layers "F.Cu" "B.Cu") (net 13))
 (segment (start 36.5 150.85) (end 35.15 149.5) (width 0.2) (layer "B.Cu") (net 13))
 (segment (start 36.5 153.7) (end 36.5 150.85) (width 0.2) (layer "B.Cu") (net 13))
 (segment (start 35.15 149.5) (end 32.4 149.5) (width 0.2) (layer "B.Cu") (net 13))
 (segment (start 34.84856 161.744949) (end 35.02354 161.569969) (width 0.2) (layer "F.Cu") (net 14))
 (segment (start 33.8 158.4) (end 33.85 158.35) (width 0.2) (layer "F.Cu") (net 14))
 (segment (start 35.8375 166) (end 35.45 166) (width 0.2) (layer "F.Cu") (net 14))
 (segment (start 33 157.5) (end 32.35 157.5) (width 0.2) (layer "F.Cu") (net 14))
 (segment (start 33.85 158.35) (end 33 157.5) (width 0.2) (layer "F.Cu") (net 14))
 (segment (start 34.84856 165.39856) (end 34.84856 161.8) (width 0.2) (layer "F.Cu") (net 14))
 (segment (start 34.84856 161.8) (end 34.84856 161.744949) (width 0.2) (layer "F.Cu") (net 14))
 (segment (start 33.8 159.65) (end 33.8 158.4) (width 0.2) (layer "F.Cu") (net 14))
 (segment (start 35.45 166) (end 34.84856 165.39856) (width 0.2) (layer "F.Cu") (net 14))
 (via (at 35.02354 161.569969) (size 0.55) (drill 0.3) (layers "F.Cu" "B.Cu") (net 14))
 (via (at 33.8 159.65) (size 0.55) (drill 0.3) (layers "F.Cu" "B.Cu") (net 14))
 (segment (start 35.02354 161.569969) (end 35.02354 160.87354) (width 0.2) (layer "B.Cu") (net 14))
 (segment (start 35.02354 160.87354) (end 33.8 159.65) (width 0.2) (layer "B.Cu") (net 14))
 (segment (start 43.412029 155.175489) (end 43.887971 155.175489) (width 0.2) (layer "F.Cu") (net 9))
 (segment (start 43.887971 155.175489) (end 44.212482 155.5) (width 0.2) (layer "F.Cu") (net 9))
 (segment (start 38.1 165.3375) (end 38.1 164.85) (width 0.2) (layer "F.Cu") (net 9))
 (segment (start 44.212482 155.5) (end 48.65 155.5) (width 0.2) (layer "F.Cu") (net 9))
 (segment (start 43.075489 155.512029) (end 43.412029 155.175489) (width 0.2) (layer "F.Cu") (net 9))
 (segment (start 43.075489 159.874511) (end 43.075489 155.512029) (width 0.2) (layer "F.Cu") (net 9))
 (segment (start 38.1 164.85) (end 43.075489 159.874511) (width 0.2) (layer "F.Cu") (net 9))
 (segment (start 45.5 153.5) (end 47.4 153.5) (width 0.2) (layer "F.Cu") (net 8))
 (segment (start 43.65 159.865006) (end 43.65 155.75) (width 0.2) (layer "F.Cu") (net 8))
 (segment (start 39.45 164.065006) (end 43.65 159.865006) (width 0.2) (layer "F.Cu") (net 8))
 (segment (start 45.3 153.7) (end 45.5 153.5) (width 0.2) (layer "F.Cu") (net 8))
 (segment (start 38.7625 166) (end 39.35 166) (width 0.2) (layer "F.Cu") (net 8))
 (segment (start 39.45 165.9) (end 39.45 164.065006) (width 0.2) (layer "F.Cu") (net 8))
 (segment (start 39.35 166) (end 39.45 165.9) (width 0.2) (layer "F.Cu") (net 8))
 (via (at 43.65 155.75) (size 0.55) (drill 0.3) (layers "F.Cu" "B.Cu") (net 8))
 (via (at 45.3 153.7) (size 0.55) (drill 0.3) (layers "F.Cu" "B.Cu") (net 8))
 (segment (start 43.65 155.75) (end 43.65 155.35) (width 0.2) (layer "B.Cu") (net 8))
 (segment (start 43.65 155.35) (end 45.3 153.7) (width 0.2) (layer "B.Cu") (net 8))
 (segment (start 44.9 173.75) (end 45.15 174) (width 0.2) (layer "F.Cu") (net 6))
 (segment (start 45.15 174) (end 48.65 174) (width 0.2) (layer "F.Cu") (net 6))
 (segment (start 38.7625 166.8) (end 44.2 166.8) (width 0.2) (layer "F.Cu") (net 6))
 (segment (start 44.2 166.8) (end 44.45 167.05) (width 0.2) (layer "F.Cu") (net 6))
 (via (at 44.9 173.75) (size 0.55) (drill 0.3) (layers "F.Cu" "B.Cu") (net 6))
 (via (at 44.45 167.05) (size 0.55) (drill 0.3) (layers "F.Cu" "B.Cu") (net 6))
 (segment (start 44.45 167.05) (end 44.45 173.3) (width 0.2) (layer "B.Cu") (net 6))
 (segment (start 44.45 173.3) (end 44.9 173.75) (width 0.2) (layer "B.Cu") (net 6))
 (segment (start 42.9 166.4) (end 38.7625 166.4) (width 0.2) (layer "F.Cu") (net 7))
 (segment (start 46.7245 164.95) (end 44.35 164.95) (width 0.2) (layer "F.Cu") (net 7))
 (segment (start 44.35 164.95) (end 42.9 166.4) (width 0.2) (layer "F.Cu") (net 7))
 (via (at 46.7245 164.95) (size 0.55) (drill 0.3) (layers "F.Cu" "B.Cu") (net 7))
 (segment (start 46.7245 165.0745) (end 46.7245 164.95) (width 0.2) (layer "B.Cu") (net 7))
 (segment (start 46.75 165.1) (end 46.7245 165.0745) (width 0.2) (layer "B.Cu") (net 7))
 (segment (start 47.65 166) (end 46.75 165.1) (width 0.2) (layer "B.Cu") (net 7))
 (segment (start 48.6 166) (end 47.65 166) (width 0.2) (layer "B.Cu") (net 7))
 (segment (start 44.2755 172) (end 43.8755 171.6) (width 0.2) (layer "F.Cu") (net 5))
 (segment (start 43.560147 167.19952) (end 38.76298 167.19952) (width 0.2) (layer "F.Cu") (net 5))
 (segment (start 48.65 172) (end 44.2755 172) (width 0.2) (layer "F.Cu") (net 5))
 (segment (start 38.76298 167.19952) (end 38.7625 167.2) (width 0.2) (layer "F.Cu") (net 5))
 (segment (start 43.826376 167.465749) (end 43.560147 167.19952) (width 0.2) (layer "F.Cu") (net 5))
 (via (at 43.8755 171.6) (size 0.55) (drill 0.3) (layers "F.Cu" "B.Cu") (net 5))
 (via (at 43.826376 167.465749) (size 0.55) (drill 0.3) (layers "F.Cu" "B.Cu") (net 5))
 (segment (start 43.8755 171.6) (end 43.826376 171.550876) (width 0.2) (layer "B.Cu") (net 5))
 (segment (start 43.826376 171.550876) (end 43.826376 167.465749) (width 0.2) (layer "B.Cu") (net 5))
 (segment (start 45.45 170) (end 47.4 170) (width 0.2) (layer "F.Cu") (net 4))
 (segment (start 38.7625 167.6) (end 43.05 167.6) (width 0.2) (layer "F.Cu") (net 4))
 (segment (start 43.05 167.6) (end 45.45 170) (width 0.2) (layer "F.Cu") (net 4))
 (segment (start 34.44904 161.328432) (end 35.263736 160.513736) (width 0.2) (layer "F.Cu") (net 15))
 (segment (start 35.25 166.4) (end 34.44904 165.59904) (width 0.2) (layer "F.Cu") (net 15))
 (segment (start 35.263736 160.513736) (end 35.277472 160.5) (width 0.2) (layer "F.Cu") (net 15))
 (segment (start 34.44904 165.59904) (end 34.44904 161.8) (width 0.2) (layer "F.Cu") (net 15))
 (segment (start 33.6 155.5) (end 32.35 155.5) (width 0.2) (layer "F.Cu") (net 15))
 (segment (start 34.44904 161.8) (end 34.44904 161.328432) (width 0.2) (layer "F.Cu") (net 15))
 (segment (start 34.443767 159.143767) (end 34.443767 156.343767) (width 0.2) (layer "F.Cu") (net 15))
 (segment (start 34.443767 156.343767) (end 33.6 155.5) (width 0.2) (layer "F.Cu") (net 15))
 (segment (start 35.277472 160.5) (end 35.55 160.5) (width 0.2) (layer "F.Cu") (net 15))
 (segment (start 35.8375 166.4) (end 35.25 166.4) (width 0.2) (layer "F.Cu") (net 15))
 (via (at 35.55 160.5) (size 0.55) (drill 0.3) (layers "F.Cu" "B.Cu") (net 15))
 (via (at 34.443767 159.143767) (size 0.55) (drill 0.3) (layers "F.Cu" "B.Cu") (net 15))
 (segment (start 35.55 160.5) (end 35.55 160.25) (width 0.2) (layer "B.Cu") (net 15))
 (segment (start 35.55 160.25) (end 34.443767 159.143767) (width 0.2) (layer "B.Cu") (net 15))
 (segment (start 35.2 158.35) (end 35.2 154.4) (width 0.2) (layer "F.Cu") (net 16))
 (segment (start 34.04952 161.7) (end 34.04952 161.162946) (width 0.2) (layer "F.Cu") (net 16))
 (segment (start 34.04952 161.162946) (end 35.756233 159.456233) (width 0.2) (layer "F.Cu") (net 16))
 (segment (start 34.04952 165.79952) (end 34.04952 161.7) (width 0.2) (layer "F.Cu") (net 16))
 (segment (start 35.2 154.4) (end 34.3 153.5) (width 0.2) (layer "F.Cu") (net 16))
 (segment (start 34.3 153.5) (end 33.6 153.5) (width 0.2) (layer "F.Cu") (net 16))
 (segment (start 35.05 166.8) (end 34.04952 165.79952) (width 0.2) (layer "F.Cu") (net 16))
 (segment (start 35.8375 166.8) (end 35.05 166.8) (width 0.2) (layer "F.Cu") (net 16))
 (via (at 35.2 158.35) (size 0.55) (drill 0.3) (layers "F.Cu" "B.Cu") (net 16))
 (via (at 35.756233 159.456233) (size 0.55) (drill 0.3) (layers "F.Cu" "B.Cu") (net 16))
 (segment (start 35.756233 159.456233) (end 35.756233 158.906233) (width 0.2) (layer "B.Cu") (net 16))
 (segment (start 35.756233 158.906233) (end 35.2 158.35) (width 0.2) (layer "B.Cu") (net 16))
 (segment (start 33.65 166.05) (end 33.65 160.75) (width 0.2) (layer "F.Cu") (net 17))
 (segment (start 35.85 152.9) (end 34.45 151.5) (width 0.2) (layer "F.Cu") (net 17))
 (segment (start 35.85 158.55) (end 35.85 152.9) (width 0.2) (layer "F.Cu") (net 17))
 (segment (start 34.45 151.5) (end 33.6 151.5) (width 0.2) (layer "F.Cu") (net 17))
 (segment (start 35.8375 167.2) (end 34.8 167.2) (width 0.2) (layer "F.Cu") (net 17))
 (segment (start 34.8 167.2) (end 33.65 166.05) (width 0.2) (layer "F.Cu") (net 17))
 (segment (start 33.65 160.75) (end 35.85 158.55) (width 0.2) (layer "F.Cu") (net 17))
 (segment (start 34.225 168.075) (end 34.7 167.6) (width 0.2) (layer "F.Cu") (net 3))
 (segment (start 34.7 167.6) (end 35.8375 167.6) (width 0.2) (layer "F.Cu") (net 3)))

